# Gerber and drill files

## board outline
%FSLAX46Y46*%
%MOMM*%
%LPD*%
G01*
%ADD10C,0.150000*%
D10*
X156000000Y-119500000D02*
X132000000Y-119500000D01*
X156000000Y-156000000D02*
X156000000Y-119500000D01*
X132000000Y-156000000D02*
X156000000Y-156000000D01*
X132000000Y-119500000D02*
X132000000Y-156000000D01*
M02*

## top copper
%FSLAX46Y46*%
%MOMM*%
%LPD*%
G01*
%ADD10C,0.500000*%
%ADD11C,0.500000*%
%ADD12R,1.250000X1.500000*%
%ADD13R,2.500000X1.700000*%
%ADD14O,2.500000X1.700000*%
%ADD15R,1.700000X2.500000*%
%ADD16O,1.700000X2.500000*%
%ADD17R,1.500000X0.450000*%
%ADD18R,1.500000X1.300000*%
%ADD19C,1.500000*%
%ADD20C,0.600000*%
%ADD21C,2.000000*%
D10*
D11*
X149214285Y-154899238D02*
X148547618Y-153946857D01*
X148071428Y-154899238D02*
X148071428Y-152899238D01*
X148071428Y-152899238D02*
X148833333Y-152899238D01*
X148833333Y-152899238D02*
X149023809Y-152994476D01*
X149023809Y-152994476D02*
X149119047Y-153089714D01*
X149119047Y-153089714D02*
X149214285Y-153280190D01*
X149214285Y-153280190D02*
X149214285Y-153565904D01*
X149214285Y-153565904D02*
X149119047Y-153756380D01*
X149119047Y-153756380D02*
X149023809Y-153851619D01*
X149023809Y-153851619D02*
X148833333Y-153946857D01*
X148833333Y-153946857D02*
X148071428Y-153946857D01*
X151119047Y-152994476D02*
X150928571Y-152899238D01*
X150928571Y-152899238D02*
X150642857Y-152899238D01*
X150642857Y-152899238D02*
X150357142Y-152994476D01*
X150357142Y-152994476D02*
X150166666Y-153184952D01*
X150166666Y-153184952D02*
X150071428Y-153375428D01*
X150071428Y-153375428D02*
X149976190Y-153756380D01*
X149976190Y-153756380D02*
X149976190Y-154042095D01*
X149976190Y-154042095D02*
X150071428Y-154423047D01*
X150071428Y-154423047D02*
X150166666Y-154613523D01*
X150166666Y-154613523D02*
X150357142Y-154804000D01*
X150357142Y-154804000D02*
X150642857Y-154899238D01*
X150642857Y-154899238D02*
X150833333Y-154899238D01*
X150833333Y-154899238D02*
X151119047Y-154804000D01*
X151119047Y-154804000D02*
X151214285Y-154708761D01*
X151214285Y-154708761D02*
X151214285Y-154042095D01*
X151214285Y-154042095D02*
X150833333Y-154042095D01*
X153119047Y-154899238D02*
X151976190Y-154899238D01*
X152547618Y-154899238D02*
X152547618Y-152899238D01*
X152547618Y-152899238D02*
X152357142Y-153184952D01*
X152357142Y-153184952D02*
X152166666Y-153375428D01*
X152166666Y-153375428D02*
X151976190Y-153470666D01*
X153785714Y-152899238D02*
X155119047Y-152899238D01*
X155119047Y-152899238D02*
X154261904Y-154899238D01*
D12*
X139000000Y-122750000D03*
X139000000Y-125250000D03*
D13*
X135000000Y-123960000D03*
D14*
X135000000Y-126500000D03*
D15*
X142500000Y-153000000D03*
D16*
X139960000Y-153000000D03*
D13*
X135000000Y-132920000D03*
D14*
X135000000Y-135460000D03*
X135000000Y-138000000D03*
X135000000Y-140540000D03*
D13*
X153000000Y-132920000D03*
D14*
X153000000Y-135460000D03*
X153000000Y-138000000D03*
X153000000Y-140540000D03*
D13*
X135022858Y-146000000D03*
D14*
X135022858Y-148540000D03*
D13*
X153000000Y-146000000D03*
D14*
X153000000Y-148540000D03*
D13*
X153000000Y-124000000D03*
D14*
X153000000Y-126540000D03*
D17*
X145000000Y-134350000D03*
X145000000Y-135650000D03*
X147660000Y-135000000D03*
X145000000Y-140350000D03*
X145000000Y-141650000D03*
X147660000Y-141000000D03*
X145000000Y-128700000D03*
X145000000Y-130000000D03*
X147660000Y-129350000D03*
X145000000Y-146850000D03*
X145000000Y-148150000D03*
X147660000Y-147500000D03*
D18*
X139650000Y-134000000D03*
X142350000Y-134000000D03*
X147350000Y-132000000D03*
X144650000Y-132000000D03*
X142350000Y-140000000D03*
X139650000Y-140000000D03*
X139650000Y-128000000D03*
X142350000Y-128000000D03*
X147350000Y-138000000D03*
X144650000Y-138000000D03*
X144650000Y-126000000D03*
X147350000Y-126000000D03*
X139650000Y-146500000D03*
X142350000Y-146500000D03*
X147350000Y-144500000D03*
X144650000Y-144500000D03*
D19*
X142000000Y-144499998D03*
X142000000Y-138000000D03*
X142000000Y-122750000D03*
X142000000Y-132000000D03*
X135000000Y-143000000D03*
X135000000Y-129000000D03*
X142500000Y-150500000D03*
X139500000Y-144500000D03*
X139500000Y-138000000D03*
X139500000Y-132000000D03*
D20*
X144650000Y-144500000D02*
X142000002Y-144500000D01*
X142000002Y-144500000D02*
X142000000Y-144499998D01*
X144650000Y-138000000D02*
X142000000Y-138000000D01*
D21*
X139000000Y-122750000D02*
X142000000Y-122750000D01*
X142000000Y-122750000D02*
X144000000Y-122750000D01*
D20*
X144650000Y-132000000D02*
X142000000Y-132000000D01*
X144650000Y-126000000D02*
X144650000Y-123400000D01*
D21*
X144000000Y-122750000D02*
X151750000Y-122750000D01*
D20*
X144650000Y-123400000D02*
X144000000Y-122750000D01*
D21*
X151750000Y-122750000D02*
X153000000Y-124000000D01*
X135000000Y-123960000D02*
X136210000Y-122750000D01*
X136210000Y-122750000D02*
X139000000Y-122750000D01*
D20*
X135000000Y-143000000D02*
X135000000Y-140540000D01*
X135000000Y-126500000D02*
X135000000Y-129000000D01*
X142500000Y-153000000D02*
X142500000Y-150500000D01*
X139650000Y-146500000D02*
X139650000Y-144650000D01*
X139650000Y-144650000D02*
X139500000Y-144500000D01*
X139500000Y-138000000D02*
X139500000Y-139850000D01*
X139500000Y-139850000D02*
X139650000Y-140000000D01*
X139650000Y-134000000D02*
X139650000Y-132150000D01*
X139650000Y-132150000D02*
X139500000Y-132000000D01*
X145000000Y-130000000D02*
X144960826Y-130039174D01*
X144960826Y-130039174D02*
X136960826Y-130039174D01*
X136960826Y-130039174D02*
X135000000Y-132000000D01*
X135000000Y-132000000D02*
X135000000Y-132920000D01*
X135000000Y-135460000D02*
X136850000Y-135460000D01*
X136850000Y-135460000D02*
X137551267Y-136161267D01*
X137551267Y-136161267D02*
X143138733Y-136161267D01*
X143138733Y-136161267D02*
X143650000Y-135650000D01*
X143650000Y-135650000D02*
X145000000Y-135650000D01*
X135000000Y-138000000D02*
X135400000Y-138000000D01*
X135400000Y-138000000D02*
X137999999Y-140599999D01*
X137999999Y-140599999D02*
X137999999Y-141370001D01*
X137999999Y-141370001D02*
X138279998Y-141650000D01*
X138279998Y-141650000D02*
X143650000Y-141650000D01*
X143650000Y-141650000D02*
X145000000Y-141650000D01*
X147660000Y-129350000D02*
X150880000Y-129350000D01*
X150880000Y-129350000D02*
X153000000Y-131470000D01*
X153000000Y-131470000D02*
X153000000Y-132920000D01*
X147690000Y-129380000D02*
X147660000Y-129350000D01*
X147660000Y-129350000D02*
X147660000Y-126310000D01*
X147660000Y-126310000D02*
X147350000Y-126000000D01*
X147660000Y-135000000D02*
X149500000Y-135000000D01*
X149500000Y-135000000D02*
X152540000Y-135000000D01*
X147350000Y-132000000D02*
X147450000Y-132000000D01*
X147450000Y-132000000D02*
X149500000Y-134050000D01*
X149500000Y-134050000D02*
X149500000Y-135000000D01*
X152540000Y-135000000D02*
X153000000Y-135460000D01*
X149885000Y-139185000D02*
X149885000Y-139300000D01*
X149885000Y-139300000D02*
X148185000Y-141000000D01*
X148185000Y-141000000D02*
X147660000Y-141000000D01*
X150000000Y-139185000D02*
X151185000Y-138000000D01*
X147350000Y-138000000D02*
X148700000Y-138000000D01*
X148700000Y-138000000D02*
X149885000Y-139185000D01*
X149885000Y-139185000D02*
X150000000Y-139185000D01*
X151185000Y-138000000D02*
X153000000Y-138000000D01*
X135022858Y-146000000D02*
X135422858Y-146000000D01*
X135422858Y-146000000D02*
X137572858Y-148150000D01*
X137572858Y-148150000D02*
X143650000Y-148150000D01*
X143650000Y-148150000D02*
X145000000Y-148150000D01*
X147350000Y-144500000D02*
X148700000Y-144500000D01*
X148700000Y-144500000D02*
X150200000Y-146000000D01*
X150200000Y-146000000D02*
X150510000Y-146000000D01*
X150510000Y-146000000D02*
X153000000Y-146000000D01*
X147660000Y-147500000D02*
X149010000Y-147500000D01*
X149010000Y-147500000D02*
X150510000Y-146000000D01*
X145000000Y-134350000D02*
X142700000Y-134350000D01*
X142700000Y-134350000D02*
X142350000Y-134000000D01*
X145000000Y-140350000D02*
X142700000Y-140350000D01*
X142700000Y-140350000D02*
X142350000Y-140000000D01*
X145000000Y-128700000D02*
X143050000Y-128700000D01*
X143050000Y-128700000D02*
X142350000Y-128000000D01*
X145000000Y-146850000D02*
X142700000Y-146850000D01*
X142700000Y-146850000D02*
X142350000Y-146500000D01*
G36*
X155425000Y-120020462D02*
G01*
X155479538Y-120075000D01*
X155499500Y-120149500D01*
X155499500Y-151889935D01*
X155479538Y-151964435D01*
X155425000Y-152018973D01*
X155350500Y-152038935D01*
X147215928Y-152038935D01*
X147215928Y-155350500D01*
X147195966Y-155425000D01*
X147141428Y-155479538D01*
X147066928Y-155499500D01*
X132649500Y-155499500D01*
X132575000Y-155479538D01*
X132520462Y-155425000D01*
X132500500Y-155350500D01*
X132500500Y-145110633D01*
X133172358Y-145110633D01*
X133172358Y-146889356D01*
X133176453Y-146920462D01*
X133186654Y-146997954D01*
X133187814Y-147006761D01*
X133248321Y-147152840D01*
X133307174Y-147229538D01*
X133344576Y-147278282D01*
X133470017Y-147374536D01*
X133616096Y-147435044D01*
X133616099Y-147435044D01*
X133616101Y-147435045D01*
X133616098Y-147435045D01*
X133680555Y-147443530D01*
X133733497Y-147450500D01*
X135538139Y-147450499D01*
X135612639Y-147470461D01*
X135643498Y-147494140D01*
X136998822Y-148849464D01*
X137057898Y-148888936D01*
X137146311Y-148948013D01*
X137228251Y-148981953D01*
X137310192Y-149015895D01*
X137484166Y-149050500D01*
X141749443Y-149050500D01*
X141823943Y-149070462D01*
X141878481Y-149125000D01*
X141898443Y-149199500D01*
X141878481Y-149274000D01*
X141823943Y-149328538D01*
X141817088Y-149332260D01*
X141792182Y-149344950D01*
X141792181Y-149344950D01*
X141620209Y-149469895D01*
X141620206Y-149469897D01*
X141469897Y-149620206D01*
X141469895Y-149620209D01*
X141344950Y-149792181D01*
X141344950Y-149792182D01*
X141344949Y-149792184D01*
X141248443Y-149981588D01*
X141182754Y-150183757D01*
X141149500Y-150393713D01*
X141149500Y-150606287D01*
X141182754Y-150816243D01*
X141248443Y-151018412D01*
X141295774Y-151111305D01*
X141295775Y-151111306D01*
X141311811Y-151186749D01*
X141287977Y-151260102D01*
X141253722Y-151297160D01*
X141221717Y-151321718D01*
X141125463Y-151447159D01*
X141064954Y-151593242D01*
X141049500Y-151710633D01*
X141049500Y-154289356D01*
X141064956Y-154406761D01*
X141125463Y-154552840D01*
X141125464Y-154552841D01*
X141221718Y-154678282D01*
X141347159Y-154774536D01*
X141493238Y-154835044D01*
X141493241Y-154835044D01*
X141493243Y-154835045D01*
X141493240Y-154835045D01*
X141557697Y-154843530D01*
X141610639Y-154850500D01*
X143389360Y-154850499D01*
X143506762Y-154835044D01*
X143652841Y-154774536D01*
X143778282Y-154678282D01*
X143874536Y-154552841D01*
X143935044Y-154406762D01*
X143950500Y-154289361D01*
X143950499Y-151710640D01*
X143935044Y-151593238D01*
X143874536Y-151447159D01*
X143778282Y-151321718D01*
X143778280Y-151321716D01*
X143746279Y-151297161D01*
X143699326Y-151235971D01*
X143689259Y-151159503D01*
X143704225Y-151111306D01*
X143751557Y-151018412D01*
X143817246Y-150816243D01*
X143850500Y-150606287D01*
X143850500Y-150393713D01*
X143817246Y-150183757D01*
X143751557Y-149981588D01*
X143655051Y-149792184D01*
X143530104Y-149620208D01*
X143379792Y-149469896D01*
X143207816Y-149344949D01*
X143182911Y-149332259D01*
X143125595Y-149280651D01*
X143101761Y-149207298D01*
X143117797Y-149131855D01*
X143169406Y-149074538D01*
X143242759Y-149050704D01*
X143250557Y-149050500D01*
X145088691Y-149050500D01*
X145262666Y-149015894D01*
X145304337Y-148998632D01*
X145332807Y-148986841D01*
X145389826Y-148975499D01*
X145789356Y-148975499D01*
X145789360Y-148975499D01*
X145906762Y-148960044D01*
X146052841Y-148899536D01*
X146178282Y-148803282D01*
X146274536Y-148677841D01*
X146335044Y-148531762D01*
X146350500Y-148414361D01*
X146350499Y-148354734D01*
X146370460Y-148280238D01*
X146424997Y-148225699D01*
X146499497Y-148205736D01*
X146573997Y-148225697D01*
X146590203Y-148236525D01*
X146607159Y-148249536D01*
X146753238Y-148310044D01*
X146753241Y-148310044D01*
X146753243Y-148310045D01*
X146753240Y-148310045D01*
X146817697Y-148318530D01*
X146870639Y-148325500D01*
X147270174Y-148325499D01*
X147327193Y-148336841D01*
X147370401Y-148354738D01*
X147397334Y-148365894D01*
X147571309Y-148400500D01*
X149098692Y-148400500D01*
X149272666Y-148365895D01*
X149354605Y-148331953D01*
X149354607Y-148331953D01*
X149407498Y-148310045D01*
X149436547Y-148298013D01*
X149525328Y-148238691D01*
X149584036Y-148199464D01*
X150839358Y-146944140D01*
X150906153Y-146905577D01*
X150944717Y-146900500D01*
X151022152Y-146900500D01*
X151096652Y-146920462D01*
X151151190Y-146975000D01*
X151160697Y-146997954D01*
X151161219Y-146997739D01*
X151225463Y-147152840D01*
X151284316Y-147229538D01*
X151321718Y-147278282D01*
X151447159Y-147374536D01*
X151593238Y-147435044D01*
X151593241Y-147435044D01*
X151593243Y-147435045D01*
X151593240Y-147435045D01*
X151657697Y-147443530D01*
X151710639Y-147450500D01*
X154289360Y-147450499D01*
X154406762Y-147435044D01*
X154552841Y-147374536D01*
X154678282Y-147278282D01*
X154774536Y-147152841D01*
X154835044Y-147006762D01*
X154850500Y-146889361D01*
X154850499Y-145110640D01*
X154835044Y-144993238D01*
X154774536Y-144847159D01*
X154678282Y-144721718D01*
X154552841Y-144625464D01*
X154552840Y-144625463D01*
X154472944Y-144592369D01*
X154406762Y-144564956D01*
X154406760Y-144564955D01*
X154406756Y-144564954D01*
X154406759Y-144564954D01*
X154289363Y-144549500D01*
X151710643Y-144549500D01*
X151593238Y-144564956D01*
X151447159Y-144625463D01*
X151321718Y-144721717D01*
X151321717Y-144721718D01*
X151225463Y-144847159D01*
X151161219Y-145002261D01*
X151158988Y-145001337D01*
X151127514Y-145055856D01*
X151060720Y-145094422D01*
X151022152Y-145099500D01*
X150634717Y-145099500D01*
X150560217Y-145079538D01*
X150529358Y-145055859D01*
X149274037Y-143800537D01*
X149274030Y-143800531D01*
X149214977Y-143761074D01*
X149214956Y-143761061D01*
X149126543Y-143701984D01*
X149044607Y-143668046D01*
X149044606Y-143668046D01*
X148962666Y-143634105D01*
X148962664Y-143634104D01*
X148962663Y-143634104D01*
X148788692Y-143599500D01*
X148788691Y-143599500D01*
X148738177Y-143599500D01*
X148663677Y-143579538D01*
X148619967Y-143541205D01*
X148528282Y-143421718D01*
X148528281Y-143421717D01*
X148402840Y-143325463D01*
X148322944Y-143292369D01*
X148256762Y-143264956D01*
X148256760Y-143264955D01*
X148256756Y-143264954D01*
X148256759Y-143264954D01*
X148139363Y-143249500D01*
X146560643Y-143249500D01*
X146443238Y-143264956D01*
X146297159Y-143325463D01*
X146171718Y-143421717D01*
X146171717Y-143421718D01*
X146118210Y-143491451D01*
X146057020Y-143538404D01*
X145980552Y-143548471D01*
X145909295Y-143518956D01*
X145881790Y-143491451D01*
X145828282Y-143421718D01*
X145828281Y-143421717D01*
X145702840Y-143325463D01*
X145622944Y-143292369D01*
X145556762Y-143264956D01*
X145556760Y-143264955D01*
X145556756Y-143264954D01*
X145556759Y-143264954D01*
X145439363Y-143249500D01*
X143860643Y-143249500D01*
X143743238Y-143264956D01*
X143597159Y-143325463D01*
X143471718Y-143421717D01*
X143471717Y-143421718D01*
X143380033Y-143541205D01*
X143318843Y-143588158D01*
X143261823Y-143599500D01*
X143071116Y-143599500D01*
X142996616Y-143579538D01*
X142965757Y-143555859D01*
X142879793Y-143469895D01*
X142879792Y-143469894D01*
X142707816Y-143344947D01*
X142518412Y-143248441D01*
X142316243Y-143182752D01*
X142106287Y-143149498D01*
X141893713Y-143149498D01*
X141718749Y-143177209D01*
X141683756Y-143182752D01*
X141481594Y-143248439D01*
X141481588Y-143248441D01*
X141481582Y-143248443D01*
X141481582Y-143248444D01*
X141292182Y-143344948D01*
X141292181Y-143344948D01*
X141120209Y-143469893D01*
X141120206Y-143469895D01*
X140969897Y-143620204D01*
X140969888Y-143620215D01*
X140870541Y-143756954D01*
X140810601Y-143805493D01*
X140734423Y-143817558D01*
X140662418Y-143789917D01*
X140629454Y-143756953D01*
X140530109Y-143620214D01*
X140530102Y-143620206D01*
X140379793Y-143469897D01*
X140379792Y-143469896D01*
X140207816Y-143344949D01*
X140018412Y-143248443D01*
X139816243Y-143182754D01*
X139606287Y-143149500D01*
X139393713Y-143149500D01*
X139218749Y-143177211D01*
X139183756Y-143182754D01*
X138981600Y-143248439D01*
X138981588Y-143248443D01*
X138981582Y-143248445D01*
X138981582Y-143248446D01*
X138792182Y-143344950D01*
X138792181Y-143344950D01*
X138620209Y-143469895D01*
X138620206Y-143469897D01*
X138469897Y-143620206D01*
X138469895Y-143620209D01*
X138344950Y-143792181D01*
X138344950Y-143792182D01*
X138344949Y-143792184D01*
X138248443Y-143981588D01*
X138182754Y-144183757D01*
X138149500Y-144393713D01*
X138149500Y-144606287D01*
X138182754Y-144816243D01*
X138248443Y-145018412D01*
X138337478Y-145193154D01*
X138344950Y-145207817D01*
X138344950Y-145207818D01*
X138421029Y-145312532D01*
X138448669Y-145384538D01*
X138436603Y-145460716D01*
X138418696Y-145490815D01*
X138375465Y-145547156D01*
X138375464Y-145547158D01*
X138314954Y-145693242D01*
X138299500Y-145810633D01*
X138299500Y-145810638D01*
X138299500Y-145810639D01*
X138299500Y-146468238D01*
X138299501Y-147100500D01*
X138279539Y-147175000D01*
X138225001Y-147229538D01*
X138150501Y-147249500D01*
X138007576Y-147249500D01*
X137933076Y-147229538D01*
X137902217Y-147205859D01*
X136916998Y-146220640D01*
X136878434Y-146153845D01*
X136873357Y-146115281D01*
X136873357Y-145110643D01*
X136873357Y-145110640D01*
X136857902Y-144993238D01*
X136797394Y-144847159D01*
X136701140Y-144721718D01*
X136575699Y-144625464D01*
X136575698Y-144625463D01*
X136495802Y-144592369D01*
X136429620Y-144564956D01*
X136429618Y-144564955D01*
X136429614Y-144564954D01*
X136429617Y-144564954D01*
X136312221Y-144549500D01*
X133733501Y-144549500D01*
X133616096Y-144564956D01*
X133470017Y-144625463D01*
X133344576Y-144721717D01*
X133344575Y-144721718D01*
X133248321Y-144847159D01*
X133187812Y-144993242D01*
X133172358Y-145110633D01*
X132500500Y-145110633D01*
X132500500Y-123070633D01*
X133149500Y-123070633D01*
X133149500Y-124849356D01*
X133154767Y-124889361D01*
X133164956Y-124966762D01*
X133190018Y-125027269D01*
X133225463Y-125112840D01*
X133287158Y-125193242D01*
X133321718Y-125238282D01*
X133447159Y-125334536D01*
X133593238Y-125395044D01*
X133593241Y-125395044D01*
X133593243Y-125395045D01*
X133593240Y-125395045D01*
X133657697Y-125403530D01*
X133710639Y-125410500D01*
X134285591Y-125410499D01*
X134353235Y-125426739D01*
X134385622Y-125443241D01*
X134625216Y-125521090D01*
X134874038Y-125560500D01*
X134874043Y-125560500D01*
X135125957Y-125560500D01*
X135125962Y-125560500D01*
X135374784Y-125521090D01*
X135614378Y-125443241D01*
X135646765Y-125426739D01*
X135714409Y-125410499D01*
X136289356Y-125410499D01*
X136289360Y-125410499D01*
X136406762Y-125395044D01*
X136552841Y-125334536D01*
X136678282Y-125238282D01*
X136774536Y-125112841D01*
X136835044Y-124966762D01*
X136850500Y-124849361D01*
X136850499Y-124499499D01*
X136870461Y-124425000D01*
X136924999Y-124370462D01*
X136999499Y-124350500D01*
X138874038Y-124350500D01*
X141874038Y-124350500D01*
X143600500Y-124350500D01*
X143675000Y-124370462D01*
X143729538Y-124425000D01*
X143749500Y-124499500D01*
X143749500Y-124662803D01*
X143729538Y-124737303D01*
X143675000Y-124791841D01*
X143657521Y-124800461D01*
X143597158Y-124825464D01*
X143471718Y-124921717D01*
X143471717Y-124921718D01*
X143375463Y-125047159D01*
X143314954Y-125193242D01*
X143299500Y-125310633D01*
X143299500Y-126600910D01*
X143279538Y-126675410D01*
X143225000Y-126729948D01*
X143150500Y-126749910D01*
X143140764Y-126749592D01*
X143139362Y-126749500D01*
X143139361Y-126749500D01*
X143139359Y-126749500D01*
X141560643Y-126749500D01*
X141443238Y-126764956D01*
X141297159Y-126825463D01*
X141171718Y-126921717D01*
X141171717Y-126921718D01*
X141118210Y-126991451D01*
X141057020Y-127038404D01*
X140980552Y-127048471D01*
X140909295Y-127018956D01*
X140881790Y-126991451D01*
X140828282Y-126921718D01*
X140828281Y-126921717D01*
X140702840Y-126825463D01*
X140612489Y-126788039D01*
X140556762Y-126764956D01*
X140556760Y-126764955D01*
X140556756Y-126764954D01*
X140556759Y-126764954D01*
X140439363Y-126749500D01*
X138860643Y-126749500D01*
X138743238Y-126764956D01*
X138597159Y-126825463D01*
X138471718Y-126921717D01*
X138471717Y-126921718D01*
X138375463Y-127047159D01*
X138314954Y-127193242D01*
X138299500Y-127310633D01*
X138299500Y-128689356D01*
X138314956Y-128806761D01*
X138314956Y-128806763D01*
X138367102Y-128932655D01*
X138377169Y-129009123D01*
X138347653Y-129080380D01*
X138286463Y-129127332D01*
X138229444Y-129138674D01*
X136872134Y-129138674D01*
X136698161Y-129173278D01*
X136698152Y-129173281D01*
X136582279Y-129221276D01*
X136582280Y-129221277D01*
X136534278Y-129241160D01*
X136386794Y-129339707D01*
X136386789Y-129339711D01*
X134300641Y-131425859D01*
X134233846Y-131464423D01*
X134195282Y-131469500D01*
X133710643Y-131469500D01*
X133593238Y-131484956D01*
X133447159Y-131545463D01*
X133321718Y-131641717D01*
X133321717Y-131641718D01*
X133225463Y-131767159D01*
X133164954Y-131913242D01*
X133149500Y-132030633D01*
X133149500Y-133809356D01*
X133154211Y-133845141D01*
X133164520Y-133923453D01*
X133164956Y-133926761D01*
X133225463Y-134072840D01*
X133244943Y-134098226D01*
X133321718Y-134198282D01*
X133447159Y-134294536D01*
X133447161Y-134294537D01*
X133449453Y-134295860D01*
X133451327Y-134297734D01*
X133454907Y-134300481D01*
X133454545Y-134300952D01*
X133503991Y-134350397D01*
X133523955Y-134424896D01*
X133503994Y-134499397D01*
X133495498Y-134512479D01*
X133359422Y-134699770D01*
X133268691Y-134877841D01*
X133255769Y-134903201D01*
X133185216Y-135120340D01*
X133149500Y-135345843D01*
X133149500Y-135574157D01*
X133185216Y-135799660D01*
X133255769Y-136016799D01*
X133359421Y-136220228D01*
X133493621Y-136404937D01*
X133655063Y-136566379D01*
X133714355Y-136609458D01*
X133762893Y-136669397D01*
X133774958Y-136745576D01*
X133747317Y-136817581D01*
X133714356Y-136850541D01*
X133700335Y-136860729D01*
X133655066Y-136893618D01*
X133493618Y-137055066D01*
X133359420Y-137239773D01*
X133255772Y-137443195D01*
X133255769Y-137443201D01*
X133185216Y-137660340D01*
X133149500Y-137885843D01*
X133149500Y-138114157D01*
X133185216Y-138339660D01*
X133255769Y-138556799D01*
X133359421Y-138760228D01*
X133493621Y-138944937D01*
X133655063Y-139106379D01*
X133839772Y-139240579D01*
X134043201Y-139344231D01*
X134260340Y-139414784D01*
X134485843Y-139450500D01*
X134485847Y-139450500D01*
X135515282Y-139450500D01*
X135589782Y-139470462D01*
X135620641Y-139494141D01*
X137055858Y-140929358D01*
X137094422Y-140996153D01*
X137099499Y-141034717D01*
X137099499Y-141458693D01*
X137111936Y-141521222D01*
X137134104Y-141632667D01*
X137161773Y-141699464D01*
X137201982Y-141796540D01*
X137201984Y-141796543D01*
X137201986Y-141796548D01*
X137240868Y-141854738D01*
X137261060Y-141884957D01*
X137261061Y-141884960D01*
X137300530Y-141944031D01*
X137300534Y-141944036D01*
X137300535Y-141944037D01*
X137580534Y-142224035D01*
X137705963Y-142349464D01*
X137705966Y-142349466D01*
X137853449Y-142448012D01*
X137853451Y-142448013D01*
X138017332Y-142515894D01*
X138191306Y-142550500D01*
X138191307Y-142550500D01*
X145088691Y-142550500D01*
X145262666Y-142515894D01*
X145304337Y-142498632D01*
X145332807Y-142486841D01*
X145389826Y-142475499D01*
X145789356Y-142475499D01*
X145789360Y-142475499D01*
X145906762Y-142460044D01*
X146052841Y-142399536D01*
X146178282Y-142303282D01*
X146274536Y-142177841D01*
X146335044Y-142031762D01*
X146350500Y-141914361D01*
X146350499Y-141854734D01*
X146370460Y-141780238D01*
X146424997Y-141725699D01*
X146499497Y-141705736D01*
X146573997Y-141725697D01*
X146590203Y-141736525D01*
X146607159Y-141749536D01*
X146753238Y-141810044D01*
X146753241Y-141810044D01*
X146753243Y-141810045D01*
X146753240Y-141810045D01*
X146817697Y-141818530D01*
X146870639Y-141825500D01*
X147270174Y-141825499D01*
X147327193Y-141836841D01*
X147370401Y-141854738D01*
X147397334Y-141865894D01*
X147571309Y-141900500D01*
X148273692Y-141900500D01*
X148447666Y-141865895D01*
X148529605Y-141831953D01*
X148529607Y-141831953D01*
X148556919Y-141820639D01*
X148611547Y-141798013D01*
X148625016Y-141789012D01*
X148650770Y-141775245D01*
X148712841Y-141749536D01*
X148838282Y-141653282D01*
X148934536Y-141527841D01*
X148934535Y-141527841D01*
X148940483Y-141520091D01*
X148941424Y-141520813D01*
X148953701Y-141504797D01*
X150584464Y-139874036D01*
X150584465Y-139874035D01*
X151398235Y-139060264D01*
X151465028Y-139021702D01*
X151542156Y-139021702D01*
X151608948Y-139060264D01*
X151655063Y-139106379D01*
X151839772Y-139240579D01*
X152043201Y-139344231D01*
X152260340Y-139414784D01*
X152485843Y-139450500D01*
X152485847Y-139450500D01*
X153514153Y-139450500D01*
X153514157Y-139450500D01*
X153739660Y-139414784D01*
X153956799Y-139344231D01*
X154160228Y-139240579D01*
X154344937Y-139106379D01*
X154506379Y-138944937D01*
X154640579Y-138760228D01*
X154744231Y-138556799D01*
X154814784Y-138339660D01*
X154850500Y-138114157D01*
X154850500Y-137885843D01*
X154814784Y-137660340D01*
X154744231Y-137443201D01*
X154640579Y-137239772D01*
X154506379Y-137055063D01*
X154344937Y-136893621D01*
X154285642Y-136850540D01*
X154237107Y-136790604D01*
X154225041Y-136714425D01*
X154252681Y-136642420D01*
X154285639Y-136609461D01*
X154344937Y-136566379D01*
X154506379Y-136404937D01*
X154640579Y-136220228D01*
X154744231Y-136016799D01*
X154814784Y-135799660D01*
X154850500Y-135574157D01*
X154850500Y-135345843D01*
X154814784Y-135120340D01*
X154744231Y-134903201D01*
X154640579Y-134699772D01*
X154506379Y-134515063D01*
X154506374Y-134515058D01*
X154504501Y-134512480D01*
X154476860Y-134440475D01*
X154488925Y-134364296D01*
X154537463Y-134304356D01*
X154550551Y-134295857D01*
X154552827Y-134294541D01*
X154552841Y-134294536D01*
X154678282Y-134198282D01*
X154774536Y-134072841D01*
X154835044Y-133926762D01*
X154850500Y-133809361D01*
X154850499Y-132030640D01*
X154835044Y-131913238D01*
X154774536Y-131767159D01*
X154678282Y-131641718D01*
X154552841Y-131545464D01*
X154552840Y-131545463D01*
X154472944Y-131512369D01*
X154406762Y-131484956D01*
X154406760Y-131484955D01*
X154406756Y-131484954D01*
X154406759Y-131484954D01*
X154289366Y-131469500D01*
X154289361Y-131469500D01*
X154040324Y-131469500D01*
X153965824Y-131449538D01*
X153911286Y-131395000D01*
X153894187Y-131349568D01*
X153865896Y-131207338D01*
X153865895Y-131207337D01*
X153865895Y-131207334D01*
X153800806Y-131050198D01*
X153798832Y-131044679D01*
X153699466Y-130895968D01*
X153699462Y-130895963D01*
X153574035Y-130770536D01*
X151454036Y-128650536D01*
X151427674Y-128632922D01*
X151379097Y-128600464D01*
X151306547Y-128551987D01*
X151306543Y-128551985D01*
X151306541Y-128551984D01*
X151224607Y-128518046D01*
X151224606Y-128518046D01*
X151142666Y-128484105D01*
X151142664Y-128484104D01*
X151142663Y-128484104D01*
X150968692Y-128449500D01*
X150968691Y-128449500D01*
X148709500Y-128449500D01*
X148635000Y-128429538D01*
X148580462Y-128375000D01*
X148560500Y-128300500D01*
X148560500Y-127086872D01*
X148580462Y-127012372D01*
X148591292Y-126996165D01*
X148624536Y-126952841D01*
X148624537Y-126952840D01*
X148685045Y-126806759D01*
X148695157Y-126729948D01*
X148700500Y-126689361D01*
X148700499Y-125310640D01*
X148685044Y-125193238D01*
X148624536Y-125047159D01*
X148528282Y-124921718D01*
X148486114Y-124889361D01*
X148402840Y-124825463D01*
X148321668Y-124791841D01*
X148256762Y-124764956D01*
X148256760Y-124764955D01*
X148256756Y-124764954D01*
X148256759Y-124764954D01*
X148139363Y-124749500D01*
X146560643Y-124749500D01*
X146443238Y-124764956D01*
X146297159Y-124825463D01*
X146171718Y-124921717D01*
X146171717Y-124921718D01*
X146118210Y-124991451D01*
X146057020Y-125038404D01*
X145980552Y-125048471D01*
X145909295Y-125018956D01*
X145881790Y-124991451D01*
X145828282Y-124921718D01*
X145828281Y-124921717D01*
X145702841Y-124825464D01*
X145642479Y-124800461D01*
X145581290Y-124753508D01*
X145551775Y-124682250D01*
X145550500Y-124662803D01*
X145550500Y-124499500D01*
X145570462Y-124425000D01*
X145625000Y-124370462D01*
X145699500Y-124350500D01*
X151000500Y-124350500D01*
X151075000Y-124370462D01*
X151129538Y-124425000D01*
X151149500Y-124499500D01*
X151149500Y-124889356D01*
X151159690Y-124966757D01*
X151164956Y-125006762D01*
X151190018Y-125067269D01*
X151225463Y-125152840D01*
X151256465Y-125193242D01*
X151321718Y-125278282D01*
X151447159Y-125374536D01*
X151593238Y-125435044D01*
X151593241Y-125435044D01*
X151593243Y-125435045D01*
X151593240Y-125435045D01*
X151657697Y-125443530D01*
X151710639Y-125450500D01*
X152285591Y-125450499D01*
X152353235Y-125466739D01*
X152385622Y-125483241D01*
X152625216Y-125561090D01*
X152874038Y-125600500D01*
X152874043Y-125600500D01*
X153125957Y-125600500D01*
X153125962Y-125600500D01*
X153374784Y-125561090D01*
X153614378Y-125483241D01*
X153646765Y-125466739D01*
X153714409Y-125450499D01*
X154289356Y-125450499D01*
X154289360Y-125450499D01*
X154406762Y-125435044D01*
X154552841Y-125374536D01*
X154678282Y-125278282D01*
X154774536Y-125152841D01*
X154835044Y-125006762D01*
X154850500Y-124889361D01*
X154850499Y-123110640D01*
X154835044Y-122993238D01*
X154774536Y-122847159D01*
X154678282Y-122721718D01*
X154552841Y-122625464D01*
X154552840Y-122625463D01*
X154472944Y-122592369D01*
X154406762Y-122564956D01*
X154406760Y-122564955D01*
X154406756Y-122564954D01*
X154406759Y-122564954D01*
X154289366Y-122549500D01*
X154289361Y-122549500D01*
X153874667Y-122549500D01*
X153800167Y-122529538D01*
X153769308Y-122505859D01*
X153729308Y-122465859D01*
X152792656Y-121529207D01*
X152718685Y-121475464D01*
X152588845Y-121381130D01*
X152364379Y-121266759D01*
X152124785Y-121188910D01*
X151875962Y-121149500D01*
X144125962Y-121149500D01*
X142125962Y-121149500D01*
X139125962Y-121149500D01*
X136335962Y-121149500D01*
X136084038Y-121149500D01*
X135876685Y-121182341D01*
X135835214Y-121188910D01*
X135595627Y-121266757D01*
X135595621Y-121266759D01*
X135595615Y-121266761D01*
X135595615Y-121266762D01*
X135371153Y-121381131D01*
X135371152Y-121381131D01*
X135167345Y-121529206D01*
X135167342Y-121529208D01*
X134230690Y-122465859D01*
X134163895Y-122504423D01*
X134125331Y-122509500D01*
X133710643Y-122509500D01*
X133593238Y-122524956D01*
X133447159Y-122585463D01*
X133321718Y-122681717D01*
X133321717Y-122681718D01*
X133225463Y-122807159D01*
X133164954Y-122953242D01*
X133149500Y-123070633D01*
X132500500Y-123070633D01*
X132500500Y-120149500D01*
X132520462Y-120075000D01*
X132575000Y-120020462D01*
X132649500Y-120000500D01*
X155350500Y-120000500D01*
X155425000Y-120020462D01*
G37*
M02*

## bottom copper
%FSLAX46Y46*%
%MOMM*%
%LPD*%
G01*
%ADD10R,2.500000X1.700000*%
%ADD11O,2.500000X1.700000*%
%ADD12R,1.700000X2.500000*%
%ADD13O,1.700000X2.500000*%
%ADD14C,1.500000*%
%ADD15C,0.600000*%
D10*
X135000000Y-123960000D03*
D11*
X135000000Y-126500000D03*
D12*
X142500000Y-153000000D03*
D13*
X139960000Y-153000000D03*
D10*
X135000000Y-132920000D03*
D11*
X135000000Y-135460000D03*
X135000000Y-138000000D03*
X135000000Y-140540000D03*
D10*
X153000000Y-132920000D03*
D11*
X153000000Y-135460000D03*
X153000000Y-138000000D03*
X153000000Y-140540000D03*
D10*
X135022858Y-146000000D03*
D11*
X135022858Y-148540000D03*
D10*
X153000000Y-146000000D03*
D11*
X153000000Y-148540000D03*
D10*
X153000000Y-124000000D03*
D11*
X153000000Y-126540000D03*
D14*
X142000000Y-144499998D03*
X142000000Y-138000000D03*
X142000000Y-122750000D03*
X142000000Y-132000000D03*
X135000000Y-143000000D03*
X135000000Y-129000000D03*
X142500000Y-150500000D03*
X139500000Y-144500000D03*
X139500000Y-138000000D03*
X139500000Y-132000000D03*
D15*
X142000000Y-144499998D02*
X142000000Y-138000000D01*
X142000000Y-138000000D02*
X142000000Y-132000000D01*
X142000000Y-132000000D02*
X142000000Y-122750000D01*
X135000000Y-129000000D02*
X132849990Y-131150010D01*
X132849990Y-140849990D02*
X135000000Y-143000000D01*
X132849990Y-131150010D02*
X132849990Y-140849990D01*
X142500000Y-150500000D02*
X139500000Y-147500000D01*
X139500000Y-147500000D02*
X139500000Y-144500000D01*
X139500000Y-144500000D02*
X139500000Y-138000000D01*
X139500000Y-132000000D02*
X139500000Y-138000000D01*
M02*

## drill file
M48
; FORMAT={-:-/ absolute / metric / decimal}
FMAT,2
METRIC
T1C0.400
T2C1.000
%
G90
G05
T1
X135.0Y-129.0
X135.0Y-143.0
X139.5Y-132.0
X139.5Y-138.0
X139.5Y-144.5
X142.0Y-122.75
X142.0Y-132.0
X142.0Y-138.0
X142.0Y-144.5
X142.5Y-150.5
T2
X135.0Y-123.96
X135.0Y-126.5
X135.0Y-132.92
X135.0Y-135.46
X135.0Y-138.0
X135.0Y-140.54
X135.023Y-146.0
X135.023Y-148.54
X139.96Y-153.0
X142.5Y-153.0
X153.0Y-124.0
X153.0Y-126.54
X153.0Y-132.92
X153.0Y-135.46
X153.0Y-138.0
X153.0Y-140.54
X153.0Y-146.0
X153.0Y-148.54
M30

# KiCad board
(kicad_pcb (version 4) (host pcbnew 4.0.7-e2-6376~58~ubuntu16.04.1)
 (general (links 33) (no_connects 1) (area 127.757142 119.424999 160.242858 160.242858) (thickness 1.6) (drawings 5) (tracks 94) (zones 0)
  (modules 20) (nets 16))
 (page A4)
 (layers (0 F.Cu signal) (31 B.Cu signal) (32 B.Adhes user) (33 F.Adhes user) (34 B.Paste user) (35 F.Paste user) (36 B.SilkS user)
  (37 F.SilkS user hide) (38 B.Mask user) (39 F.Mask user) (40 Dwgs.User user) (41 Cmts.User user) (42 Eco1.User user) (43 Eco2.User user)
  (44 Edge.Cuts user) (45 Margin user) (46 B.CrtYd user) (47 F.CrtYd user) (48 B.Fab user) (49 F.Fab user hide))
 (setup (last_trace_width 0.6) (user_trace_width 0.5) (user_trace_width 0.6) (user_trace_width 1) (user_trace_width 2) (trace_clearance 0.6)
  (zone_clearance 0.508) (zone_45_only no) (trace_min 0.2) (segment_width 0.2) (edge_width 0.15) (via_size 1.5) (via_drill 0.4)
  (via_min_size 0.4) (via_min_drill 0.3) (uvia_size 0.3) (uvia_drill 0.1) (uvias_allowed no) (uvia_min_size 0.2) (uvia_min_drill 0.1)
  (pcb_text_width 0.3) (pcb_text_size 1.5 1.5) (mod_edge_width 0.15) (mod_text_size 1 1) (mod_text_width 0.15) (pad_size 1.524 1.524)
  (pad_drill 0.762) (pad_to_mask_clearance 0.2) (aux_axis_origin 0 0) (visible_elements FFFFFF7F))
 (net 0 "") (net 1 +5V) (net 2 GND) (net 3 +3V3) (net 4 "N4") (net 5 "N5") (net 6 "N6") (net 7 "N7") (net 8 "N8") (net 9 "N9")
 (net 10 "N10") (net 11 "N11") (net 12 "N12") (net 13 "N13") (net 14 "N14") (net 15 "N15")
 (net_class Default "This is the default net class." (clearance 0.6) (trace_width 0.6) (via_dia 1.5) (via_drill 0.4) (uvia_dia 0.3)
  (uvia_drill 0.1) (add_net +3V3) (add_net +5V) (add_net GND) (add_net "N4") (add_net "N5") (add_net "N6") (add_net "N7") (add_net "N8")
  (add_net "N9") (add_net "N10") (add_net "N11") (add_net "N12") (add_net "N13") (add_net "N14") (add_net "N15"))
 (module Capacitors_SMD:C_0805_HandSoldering (layer F.Cu) (at 139 124 270)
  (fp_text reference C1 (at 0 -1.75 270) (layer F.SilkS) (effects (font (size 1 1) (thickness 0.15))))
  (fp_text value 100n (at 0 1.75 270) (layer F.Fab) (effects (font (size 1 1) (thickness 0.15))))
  (pad 1 smd rect (at -1.25 0 270) (size 1.5 1.25) (layers F.Cu F.Paste F.Mask) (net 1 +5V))
  (pad 2 smd rect (at 1.25 0 270) (size 1.5 1.25) (layers F.Cu F.Paste F.Mask) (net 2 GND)))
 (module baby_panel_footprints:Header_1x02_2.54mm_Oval (layer F.Cu) (at 135 123.96)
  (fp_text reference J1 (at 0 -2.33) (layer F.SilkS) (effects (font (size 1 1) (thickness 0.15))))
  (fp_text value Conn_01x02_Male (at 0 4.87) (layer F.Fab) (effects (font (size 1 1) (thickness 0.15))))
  (pad 1 thru_hole rect (at 0 0) (size 2.5 1.7) (drill 1) (layers *.Cu *.Mask) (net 1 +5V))
  (pad 2 thru_hole oval (at 0 2.54) (size 2.5 1.7) (drill 1) (layers *.Cu *.Mask) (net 2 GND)))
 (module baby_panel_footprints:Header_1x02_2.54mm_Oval (layer F.Cu) (at 142.5 153 270)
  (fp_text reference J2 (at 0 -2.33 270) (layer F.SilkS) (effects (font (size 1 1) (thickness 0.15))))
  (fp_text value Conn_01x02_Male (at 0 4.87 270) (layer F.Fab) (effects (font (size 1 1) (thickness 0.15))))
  (pad 1 thru_hole rect (at 0 0 270) (size 2.5 1.7) (drill 1) (layers *.Cu *.Mask) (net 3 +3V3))
  (pad 2 thru_hole oval (at 0 2.54 270) (size 2.5 1.7) (drill 1) (layers *.Cu *.Mask) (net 2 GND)))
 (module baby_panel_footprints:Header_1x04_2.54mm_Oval (layer F.Cu) (at 135 132.92)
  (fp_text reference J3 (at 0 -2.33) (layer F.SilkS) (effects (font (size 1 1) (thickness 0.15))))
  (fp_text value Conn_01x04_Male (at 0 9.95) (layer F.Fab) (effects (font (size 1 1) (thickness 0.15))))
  (pad 1 thru_hole rect (at 0 0) (size 2.5 1.7) (drill 1) (layers *.Cu *.Mask) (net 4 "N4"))
  (pad 2 thru_hole oval (at 0 2.54) (size 2.5 1.7) (drill 1) (layers *.Cu *.Mask) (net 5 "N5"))
  (pad 3 thru_hole oval (at 0 5.08) (size 2.5 1.7) (drill 1) (layers *.Cu *.Mask) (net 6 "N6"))
  (pad 4 thru_hole oval (at 0 7.62) (size 2.5 1.7) (drill 1) (layers *.Cu *.Mask) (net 2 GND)))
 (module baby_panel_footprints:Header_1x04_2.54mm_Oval (layer F.Cu) (at 153 132.92)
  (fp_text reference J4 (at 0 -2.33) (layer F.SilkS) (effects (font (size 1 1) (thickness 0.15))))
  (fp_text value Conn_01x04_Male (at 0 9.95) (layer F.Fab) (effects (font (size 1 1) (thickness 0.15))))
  (pad 1 thru_hole rect (at 0 0) (size 2.5 1.7) (drill 1) (layers *.Cu *.Mask) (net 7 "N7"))
  (pad 2 thru_hole oval (at 0 2.54) (size 2.5 1.7) (drill 1) (layers *.Cu *.Mask) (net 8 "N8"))
  (pad 3 thru_hole oval (at 0 5.08) (size 2.5 1.7) (drill 1) (layers *.Cu *.Mask) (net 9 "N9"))
  (pad 4 thru_hole oval (at 0 7.62) (size 2.5 1.7) (drill 1) (layers *.Cu *.Mask) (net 2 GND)))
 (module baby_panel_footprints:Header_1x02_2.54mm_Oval (layer F.Cu) (at 135.022858 146)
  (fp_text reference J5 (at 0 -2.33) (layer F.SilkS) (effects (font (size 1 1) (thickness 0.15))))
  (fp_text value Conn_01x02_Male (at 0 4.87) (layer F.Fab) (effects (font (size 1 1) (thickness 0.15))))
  (pad 1 thru_hole rect (at 0 0) (size 2.5 1.7) (drill 1) (layers *.Cu *.Mask) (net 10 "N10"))
  (pad 2 thru_hole oval (at 0 2.54) (size 2.5 1.7) (drill 1) (layers *.Cu *.Mask) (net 2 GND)))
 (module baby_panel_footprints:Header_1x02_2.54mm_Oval (layer F.Cu) (at 153 146)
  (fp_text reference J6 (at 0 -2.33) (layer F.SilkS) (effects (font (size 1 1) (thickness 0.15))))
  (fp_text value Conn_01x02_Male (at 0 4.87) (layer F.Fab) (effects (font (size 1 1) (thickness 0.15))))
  (pad 1 thru_hole rect (at 0 0) (size 2.5 1.7) (drill 1) (layers *.Cu *.Mask) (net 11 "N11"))
  (pad 2 thru_hole oval (at 0 2.54) (size 2.5 1.7) (drill 1) (layers *.Cu *.Mask) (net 2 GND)))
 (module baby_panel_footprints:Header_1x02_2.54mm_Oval (layer F.Cu) (at 153 124)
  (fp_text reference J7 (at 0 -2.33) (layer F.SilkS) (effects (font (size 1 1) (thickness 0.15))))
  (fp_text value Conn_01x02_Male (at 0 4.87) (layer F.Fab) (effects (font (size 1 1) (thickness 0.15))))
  (pad 1 thru_hole rect (at 0 0) (size 2.5 1.7) (drill 1) (layers *.Cu *.Mask) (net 1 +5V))
  (pad 2 thru_hole oval (at 0 2.54) (size 2.5 1.7) (drill 1) (layers *.Cu *.Mask) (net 2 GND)))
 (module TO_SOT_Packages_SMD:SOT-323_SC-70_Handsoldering (layer F.Cu) (at 146.33 135)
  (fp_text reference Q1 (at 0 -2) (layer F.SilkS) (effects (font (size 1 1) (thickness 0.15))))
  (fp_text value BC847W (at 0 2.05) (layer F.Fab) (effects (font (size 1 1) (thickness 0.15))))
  (pad 1 smd rect (at -1.33 -0.65 270) (size 0.45 1.5) (layers F.Cu F.Paste F.Mask) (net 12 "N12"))
  (pad 2 smd rect (at -1.33 0.65 270) (size 0.45 1.5) (layers F.Cu F.Paste F.Mask) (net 5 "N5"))
  (pad 3 smd rect (at 1.33 0 270) (size 0.45 1.5) (layers F.Cu F.Paste F.Mask) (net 8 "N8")))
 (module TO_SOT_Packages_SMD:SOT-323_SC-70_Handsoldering (layer F.Cu) (at 146.33 141)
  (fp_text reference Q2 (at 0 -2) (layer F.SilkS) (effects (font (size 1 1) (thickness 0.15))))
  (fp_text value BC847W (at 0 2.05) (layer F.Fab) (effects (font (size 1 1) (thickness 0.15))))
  (pad 1 smd rect (at -1.33 -0.65 270) (size 0.45 1.5) (layers F.Cu F.Paste F.Mask) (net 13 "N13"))
  (pad 2 smd rect (at -1.33 0.65 270) (size 0.45 1.5) (layers F.Cu F.Paste F.Mask) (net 6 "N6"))
  (pad 3 smd rect (at 1.33 0 270) (size 0.45 1.5) (layers F.Cu F.Paste F.Mask) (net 9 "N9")))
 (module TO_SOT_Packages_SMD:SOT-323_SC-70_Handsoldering (layer F.Cu) (at 146.33 129.35)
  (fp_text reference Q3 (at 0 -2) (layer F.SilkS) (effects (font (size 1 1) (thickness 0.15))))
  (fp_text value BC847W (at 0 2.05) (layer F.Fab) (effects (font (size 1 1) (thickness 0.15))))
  (pad 1 smd rect (at -1.33 -0.65 270) (size 0.45 1.5) (layers F.Cu F.Paste F.Mask) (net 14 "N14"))
  (pad 2 smd rect (at -1.33 0.65 270) (size 0.45 1.5) (layers F.Cu F.Paste F.Mask) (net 4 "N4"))
  (pad 3 smd rect (at 1.33 0 270) (size 0.45 1.5) (layers F.Cu F.Paste F.Mask) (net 7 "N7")))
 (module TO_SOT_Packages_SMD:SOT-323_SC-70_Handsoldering (layer F.Cu) (at 146.33 147.5)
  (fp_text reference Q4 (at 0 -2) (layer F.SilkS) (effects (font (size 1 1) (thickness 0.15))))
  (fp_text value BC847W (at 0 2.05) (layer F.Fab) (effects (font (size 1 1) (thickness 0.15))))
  (pad 1 smd rect (at -1.33 -0.65 270) (size 0.45 1.5) (layers F.Cu F.Paste F.Mask) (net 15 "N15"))
  (pad 2 smd rect (at -1.33 0.65 270) (size 0.45 1.5) (layers F.Cu F.Paste F.Mask) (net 10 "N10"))
  (pad 3 smd rect (at 1.33 0 270) (size 0.45 1.5) (layers F.Cu F.Paste F.Mask) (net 11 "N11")))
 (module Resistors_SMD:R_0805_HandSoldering (layer F.Cu) (at 141 134)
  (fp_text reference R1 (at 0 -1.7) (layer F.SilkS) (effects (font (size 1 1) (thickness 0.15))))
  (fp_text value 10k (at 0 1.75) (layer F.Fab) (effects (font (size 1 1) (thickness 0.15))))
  (pad 1 smd rect (at -1.35 0) (size 1.5 1.3) (layers F.Cu F.Paste F.Mask) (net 3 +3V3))
  (pad 2 smd rect (at 1.35 0) (size 1.5 1.3) (layers F.Cu F.Paste F.Mask) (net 12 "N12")))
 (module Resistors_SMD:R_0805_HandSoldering (layer F.Cu) (at 146 132 180)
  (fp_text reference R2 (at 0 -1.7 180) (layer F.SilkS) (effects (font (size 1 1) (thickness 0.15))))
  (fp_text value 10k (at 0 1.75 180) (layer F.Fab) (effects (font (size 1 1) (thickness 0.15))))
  (pad 1 smd rect (at -1.35 0 180) (size 1.5 1.3) (layers F.Cu F.Paste F.Mask) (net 8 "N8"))
  (pad 2 smd rect (at 1.35 0 180) (size 1.5 1.3) (layers F.Cu F.Paste F.Mask) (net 1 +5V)))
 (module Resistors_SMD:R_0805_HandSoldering (layer F.Cu) (at 141 140 180)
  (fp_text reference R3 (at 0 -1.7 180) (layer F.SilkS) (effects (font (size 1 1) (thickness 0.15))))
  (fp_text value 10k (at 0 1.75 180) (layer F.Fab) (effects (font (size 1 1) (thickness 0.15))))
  (pad 1 smd rect (at -1.35 0 180) (size 1.5 1.3) (layers F.Cu F.Paste F.Mask) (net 13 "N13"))
  (pad 2 smd rect (at 1.35 0 180) (size 1.5 1.3) (layers F.Cu F.Paste F.Mask) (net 3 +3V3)))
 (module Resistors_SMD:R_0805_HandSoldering (layer F.Cu) (at 141 128)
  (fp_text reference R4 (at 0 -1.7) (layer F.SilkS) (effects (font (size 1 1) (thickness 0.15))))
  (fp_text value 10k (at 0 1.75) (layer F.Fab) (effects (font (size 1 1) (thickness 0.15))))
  (pad 1 smd rect (at -1.35 0) (size 1.5 1.3) (layers F.Cu F.Paste F.Mask) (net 3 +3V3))
  (pad 2 smd rect (at 1.35 0) (size 1.5 1.3) (layers F.Cu F.Paste F.Mask) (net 14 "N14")))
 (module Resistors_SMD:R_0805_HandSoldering (layer F.Cu) (at 146 138 180)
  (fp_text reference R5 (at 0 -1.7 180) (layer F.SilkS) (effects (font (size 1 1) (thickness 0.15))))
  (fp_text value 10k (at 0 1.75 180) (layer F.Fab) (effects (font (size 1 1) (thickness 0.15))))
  (pad 1 smd rect (at -1.35 0 180) (size 1.5 1.3) (layers F.Cu F.Paste F.Mask) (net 9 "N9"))
  (pad 2 smd rect (at 1.35 0 180) (size 1.5 1.3) (layers F.Cu F.Paste F.Mask) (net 1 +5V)))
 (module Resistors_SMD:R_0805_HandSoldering (layer F.Cu) (at 146 126)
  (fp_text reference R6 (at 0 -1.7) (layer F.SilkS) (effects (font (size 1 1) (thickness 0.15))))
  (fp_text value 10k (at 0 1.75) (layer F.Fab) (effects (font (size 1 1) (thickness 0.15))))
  (pad 1 smd rect (at -1.35 0) (size 1.5 1.3) (layers F.Cu F.Paste F.Mask) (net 1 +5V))
  (pad 2 smd rect (at 1.35 0) (size 1.5 1.3) (layers F.Cu F.Paste F.Mask) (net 7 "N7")))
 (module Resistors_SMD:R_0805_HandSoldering (layer F.Cu) (at 141 146.5)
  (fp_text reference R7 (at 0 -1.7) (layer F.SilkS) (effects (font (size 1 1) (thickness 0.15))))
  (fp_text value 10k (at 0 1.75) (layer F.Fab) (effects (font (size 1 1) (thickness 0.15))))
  (pad 1 smd rect (at -1.35 0) (size 1.5 1.3) (layers F.Cu F.Paste F.Mask) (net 3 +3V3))
  (pad 2 smd rect (at 1.35 0) (size 1.5 1.3) (layers F.Cu F.Paste F.Mask) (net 15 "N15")))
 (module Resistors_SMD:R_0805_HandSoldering (layer F.Cu) (at 146 144.5 180)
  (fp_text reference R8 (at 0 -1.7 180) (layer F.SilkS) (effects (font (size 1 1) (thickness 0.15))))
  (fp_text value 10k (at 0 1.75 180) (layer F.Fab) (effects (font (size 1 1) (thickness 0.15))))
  (pad 1 smd rect (at -1.35 0 180) (size 1.5 1.3) (layers F.Cu F.Paste F.Mask) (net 11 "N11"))
  (pad 2 smd rect (at 1.35 0 180) (size 1.5 1.3) (layers F.Cu F.Paste F.Mask) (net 1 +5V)))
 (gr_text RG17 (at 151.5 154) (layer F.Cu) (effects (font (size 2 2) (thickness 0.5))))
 (gr_line (start 156 119.5) (end 132 119.5) (layer Edge.Cuts) (width 0.15))
 (gr_line (start 156 156) (end 156 119.5) (layer Edge.Cuts) (width 0.15))
 (gr_line (start 132 156) (end 156 156) (layer Edge.Cuts) (width 0.15))
 (gr_line (start 132 119.5) (end 132 156) (layer Edge.Cuts) (width 0.15))
 (segment (start 142 144.499998) (end 142 138) (width 0.6) (layer B.Cu) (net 1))
 (segment (start 144.65 144.5) (end 142.000002 144.5) (width 0.6) (layer F.Cu) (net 1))
 (segment (start 142.000002 144.5) (end 142 144.499998) (width 0.6) (layer F.Cu) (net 1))
 (via (at 142 144.499998) (size 1.5) (drill 0.4) (layers F.Cu B.Cu) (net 1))
 (segment (start 142 138) (end 142 132) (width 0.6) (layer B.Cu) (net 1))
 (segment (start 144.65 138) (end 142 138) (width 0.6) (layer F.Cu) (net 1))
 (via (at 142 138) (size 1.5) (drill 0.4) (layers F.Cu B.Cu) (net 1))
 (segment (start 139 122.75) (end 142 122.75) (width 2) (layer F.Cu) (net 1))
 (segment (start 142 122.75) (end 144 122.75) (width 2) (layer F.Cu) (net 1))
 (segment (start 142 132) (end 142 122.75) (width 0.6) (layer B.Cu) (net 1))
 (via (at 142 122.75) (size 1.5) (drill 0.4) (layers F.Cu B.Cu) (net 1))
 (segment (start 144.65 132) (end 142 132) (width 0.6) (layer F.Cu) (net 1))
 (via (at 142 132) (size 1.5) (drill 0.4) (layers F.Cu B.Cu) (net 1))
 (segment (start 144.65 126) (end 144.65 123.4) (width 0.6) (layer F.Cu) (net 1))
 (segment (start 144 122.75) (end 151.75 122.75) (width 2) (layer F.Cu) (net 1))
 (segment (start 144.65 123.4) (end 144 122.75) (width 0.6) (layer F.Cu) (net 1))
 (segment (start 151.75 122.75) (end 153 124) (width 2) (layer F.Cu) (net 1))
 (segment (start 135 123.96) (end 136.21 122.75) (width 2) (layer F.Cu) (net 1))
 (segment (start 136.21 122.75) (end 139 122.75) (width 2) (layer F.Cu) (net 1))
 (segment (start 135 143) (end 135 140.54) (width 0.6) (layer F.Cu) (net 2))
 (segment (start 135 129) (end 132.84999 131.15001) (width 0.6) (layer B.Cu) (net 2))
 (segment (start 132.84999 140.84999) (end 135 143) (width 0.6) (layer B.Cu) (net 2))
 (segment (start 132.84999 131.15001) (end 132.84999 140.84999) (width 0.6) (layer B.Cu) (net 2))
 (via (at 135 143) (size 1.5) (drill 0.4) (layers F.Cu B.Cu) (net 2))
 (segment (start 135 126.5) (end 135 129) (width 0.6) (layer F.Cu) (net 2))
 (via (at 135 129) (size 1.5) (drill 0.4) (layers F.Cu B.Cu) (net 2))
 (segment (start 142.5 150.5) (end 139.5 147.5) (width 0.6) (layer B.Cu) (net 3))
 (segment (start 139.5 147.5) (end 139.5 144.5) (width 0.6) (layer B.Cu) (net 3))
 (segment (start 142.5 153) (end 142.5 150.5) (width 0.6) (layer F.Cu) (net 3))
 (via (at 142.5 150.5) (size 1.5) (drill 0.4) (layers F.Cu B.Cu) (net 3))
 (segment (start 139.5 144.5) (end 139.5 138) (width 0.6) (layer B.Cu) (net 3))
 (segment (start 139.65 146.5) (end 139.65 144.65) (width 0.6) (layer F.Cu) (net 3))
 (segment (start 139.65 144.65) (end 139.5 144.5) (width 0.6) (layer F.Cu) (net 3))
 (via (at 139.5 144.5) (size 1.5) (drill 0.4) (layers F.Cu B.Cu) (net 3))
 (segment (start 139.5 138) (end 139.5 139.85) (width 0.6) (layer F.Cu) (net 3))
 (segment (start 139.5 139.85) (end 139.65 140) (width 0.6) (layer F.Cu) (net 3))
 (segment (start 139.5 132) (end 139.5 138) (width 0.6) (layer B.Cu) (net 3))
 (via (at 139.5 138) (size 1.5) (drill 0.4) (layers F.Cu B.Cu) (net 3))
 (segment (start 139.65 134) (end 139.65 132.15) (width 0.6) (layer F.Cu) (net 3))
 (segment (start 139.65 132.15) (end 139.5 132) (width 0.6) (layer F.Cu) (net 3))
 (via (at 139.5 132) (size 1.5) (drill 0.4) (layers F.Cu B.Cu) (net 3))
 (segment (start 145 130) (end 144.960826 130.039174) (width 0.6) (layer F.Cu) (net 4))
 (segment (start 144.960826 130.039174) (end 136.960826 130.039174) (width 0.6) (layer F.Cu) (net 4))
 (segment (start 136.960826 130.039174) (end 135 132) (width 0.6) (layer F.Cu) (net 4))
 (segment (start 135 132) (end 135 132.92) (width 0.6) (layer F.Cu) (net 4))
 (segment (start 135 135.46) (end 136.85 135.46) (width 0.6) (layer F.Cu) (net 5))
 (segment (start 136.85 135.46) (end 137.551267 136.161267) (width 0.6) (layer F.Cu) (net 5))
 (segment (start 137.551267 136.161267) (end 143.138733 136.161267) (width 0.6) (layer F.Cu) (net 5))
 (segment (start 143.138733 136.161267) (end 143.65 135.65) (width 0.6) (layer F.Cu) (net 5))
 (segment (start 143.65 135.65) (end 145 135.65) (width 0.6) (layer F.Cu) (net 5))
 (segment (start 135 138) (end 135.4 138) (width 0.6) (layer F.Cu) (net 6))
 (segment (start 135.4 138) (end 137.999999 140.599999) (width 0.6) (layer F.Cu) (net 6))
 (segment (start 137.999999 140.599999) (end 137.999999 141.370001) (width 0.6) (layer F.Cu) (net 6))
 (segment (start 137.999999 141.370001) (end 138.279998 141.65) (width 0.6) (layer F.Cu) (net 6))
 (segment (start 138.279998 141.65) (end 143.65 141.65) (width 0.6) (layer F.Cu) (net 6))
 (segment (start 143.65 141.65) (end 145 141.65) (width 0.6) (layer F.Cu) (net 6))
 (segment (start 147.66 129.35) (end 150.88 129.35) (width 0.6) (layer F.Cu) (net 7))
 (segment (start 150.88 129.35) (end 153 131.47) (width 0.6) (layer F.Cu) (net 7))
 (segment (start 153 131.47) (end 153 132.92) (width 0.6) (layer F.Cu) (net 7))
 (segment (start 147.69 129.38) (end 147.66 129.35) (width 0.6) (layer F.Cu) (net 7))
 (segment (start 147.66 129.35) (end 147.66 126.31) (width 0.6) (layer F.Cu) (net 7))
 (segment (start 147.66 126.31) (end 147.35 126) (width 0.6) (layer F.Cu) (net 7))
 (segment (start 147.66 135) (end 149.5 135) (width 0.6) (layer F.Cu) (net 8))
 (segment (start 149.5 135) (end 152.54 135) (width 0.6) (layer F.Cu) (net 8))
 (segment (start 147.35 132) (end 147.45 132) (width 0.6) (layer F.Cu) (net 8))
 (segment (start 147.45 132) (end 149.5 134.05) (width 0.6) (layer F.Cu) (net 8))
 (segment (start 149.5 134.05) (end 149.5 135) (width 0.6) (layer F.Cu) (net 8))
 (segment (start 152.54 135) (end 153 135.46) (width 0.6) (layer F.Cu) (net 8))
 (segment (start 149.885 139.185) (end 149.885 139.3) (width 0.6) (layer F.Cu) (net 9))
 (segment (start 149.885 139.3) (end 148.185 141) (width 0.6) (layer F.Cu) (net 9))
 (segment (start 148.185 141) (end 147.66 141) (width 0.6) (layer F.Cu) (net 9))
 (segment (start 150 139.185) (end 151.185 138) (width 0.6) (layer F.Cu) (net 9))
 (segment (start 147.35 138) (end 148.7 138) (width 0.6) (layer F.Cu) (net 9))
 (segment (start 148.7 138) (end 149.885 139.185) (width 0.6) (layer F.Cu) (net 9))
 (segment (start 149.885 139.185) (end 150 139.185) (width 0.6) (layer F.Cu) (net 9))
 (segment (start 151.185 138) (end 153 138) (width 0.6) (layer F.Cu) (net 9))
 (segment (start 135.022858 146) (end 135.422858 146) (width 0.6) (layer F.Cu) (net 10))
 (segment (start 135.422858 146) (end 137.572858 148.15) (width 0.6) (layer F.Cu) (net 10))
 (segment (start 137.572858 148.15) (end 143.65 148.15) (width 0.6) (layer F.Cu) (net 10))
 (segment (start 143.65 148.15) (end 145 148.15) (width 0.6) (layer F.Cu) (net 10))
 (segment (start 147.35 144.5) (end 148.7 144.5) (width 0.6) (layer F.Cu) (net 11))
 (segment (start 148.7 144.5) (end 150.2 146) (width 0.6) (layer F.Cu) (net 11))
 (segment (start 150.2 146) (end 150.51 146) (width 0.6) (layer F.Cu) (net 11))
 (segment (start 150.51 146) (end 153 146) (width 0.6) (layer F.Cu) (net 11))
 (segment (start 147.66 147.5) (end 149.01 147.5) (width 0.6) (layer F.Cu) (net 11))
 (segment (start 149.01 147.5) (end 150.51 146) (width 0.6) (layer F.Cu) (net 11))
 (segment (start 145 134.35) (end 142.7 134.35) (width 0.6) (layer F.Cu) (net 12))
 (segment (start 142.7 134.35) (end 142.35 134) (width 0.6) (layer F.Cu) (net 12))
 (segment (start 145 140.35) (end 142.7 140.35) (width 0.6) (layer F.Cu) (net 13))
 (segment (start 142.7 140.35) (end 142.35 140) (width 0.6) (layer F.Cu) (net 13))
 (segment (start 145 128.7) (end 143.05 128.7) (width 0.6) (layer F.Cu) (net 14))
 (segment (start 143.05 128.7) (end 142.35 128) (width 0.6) (layer F.Cu) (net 14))
 (segment (start 145 146.85) (end 142.7 146.85) (width 0.6) (layer F.Cu) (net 15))
 (segment (start 142.7 146.85) (end 142.35 146.5) (width 0.6) (layer F.Cu) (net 15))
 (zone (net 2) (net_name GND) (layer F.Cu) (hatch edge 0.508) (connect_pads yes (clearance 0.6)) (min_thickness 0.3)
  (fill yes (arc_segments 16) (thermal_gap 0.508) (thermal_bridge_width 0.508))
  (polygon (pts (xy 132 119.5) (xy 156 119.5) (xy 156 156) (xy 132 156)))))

